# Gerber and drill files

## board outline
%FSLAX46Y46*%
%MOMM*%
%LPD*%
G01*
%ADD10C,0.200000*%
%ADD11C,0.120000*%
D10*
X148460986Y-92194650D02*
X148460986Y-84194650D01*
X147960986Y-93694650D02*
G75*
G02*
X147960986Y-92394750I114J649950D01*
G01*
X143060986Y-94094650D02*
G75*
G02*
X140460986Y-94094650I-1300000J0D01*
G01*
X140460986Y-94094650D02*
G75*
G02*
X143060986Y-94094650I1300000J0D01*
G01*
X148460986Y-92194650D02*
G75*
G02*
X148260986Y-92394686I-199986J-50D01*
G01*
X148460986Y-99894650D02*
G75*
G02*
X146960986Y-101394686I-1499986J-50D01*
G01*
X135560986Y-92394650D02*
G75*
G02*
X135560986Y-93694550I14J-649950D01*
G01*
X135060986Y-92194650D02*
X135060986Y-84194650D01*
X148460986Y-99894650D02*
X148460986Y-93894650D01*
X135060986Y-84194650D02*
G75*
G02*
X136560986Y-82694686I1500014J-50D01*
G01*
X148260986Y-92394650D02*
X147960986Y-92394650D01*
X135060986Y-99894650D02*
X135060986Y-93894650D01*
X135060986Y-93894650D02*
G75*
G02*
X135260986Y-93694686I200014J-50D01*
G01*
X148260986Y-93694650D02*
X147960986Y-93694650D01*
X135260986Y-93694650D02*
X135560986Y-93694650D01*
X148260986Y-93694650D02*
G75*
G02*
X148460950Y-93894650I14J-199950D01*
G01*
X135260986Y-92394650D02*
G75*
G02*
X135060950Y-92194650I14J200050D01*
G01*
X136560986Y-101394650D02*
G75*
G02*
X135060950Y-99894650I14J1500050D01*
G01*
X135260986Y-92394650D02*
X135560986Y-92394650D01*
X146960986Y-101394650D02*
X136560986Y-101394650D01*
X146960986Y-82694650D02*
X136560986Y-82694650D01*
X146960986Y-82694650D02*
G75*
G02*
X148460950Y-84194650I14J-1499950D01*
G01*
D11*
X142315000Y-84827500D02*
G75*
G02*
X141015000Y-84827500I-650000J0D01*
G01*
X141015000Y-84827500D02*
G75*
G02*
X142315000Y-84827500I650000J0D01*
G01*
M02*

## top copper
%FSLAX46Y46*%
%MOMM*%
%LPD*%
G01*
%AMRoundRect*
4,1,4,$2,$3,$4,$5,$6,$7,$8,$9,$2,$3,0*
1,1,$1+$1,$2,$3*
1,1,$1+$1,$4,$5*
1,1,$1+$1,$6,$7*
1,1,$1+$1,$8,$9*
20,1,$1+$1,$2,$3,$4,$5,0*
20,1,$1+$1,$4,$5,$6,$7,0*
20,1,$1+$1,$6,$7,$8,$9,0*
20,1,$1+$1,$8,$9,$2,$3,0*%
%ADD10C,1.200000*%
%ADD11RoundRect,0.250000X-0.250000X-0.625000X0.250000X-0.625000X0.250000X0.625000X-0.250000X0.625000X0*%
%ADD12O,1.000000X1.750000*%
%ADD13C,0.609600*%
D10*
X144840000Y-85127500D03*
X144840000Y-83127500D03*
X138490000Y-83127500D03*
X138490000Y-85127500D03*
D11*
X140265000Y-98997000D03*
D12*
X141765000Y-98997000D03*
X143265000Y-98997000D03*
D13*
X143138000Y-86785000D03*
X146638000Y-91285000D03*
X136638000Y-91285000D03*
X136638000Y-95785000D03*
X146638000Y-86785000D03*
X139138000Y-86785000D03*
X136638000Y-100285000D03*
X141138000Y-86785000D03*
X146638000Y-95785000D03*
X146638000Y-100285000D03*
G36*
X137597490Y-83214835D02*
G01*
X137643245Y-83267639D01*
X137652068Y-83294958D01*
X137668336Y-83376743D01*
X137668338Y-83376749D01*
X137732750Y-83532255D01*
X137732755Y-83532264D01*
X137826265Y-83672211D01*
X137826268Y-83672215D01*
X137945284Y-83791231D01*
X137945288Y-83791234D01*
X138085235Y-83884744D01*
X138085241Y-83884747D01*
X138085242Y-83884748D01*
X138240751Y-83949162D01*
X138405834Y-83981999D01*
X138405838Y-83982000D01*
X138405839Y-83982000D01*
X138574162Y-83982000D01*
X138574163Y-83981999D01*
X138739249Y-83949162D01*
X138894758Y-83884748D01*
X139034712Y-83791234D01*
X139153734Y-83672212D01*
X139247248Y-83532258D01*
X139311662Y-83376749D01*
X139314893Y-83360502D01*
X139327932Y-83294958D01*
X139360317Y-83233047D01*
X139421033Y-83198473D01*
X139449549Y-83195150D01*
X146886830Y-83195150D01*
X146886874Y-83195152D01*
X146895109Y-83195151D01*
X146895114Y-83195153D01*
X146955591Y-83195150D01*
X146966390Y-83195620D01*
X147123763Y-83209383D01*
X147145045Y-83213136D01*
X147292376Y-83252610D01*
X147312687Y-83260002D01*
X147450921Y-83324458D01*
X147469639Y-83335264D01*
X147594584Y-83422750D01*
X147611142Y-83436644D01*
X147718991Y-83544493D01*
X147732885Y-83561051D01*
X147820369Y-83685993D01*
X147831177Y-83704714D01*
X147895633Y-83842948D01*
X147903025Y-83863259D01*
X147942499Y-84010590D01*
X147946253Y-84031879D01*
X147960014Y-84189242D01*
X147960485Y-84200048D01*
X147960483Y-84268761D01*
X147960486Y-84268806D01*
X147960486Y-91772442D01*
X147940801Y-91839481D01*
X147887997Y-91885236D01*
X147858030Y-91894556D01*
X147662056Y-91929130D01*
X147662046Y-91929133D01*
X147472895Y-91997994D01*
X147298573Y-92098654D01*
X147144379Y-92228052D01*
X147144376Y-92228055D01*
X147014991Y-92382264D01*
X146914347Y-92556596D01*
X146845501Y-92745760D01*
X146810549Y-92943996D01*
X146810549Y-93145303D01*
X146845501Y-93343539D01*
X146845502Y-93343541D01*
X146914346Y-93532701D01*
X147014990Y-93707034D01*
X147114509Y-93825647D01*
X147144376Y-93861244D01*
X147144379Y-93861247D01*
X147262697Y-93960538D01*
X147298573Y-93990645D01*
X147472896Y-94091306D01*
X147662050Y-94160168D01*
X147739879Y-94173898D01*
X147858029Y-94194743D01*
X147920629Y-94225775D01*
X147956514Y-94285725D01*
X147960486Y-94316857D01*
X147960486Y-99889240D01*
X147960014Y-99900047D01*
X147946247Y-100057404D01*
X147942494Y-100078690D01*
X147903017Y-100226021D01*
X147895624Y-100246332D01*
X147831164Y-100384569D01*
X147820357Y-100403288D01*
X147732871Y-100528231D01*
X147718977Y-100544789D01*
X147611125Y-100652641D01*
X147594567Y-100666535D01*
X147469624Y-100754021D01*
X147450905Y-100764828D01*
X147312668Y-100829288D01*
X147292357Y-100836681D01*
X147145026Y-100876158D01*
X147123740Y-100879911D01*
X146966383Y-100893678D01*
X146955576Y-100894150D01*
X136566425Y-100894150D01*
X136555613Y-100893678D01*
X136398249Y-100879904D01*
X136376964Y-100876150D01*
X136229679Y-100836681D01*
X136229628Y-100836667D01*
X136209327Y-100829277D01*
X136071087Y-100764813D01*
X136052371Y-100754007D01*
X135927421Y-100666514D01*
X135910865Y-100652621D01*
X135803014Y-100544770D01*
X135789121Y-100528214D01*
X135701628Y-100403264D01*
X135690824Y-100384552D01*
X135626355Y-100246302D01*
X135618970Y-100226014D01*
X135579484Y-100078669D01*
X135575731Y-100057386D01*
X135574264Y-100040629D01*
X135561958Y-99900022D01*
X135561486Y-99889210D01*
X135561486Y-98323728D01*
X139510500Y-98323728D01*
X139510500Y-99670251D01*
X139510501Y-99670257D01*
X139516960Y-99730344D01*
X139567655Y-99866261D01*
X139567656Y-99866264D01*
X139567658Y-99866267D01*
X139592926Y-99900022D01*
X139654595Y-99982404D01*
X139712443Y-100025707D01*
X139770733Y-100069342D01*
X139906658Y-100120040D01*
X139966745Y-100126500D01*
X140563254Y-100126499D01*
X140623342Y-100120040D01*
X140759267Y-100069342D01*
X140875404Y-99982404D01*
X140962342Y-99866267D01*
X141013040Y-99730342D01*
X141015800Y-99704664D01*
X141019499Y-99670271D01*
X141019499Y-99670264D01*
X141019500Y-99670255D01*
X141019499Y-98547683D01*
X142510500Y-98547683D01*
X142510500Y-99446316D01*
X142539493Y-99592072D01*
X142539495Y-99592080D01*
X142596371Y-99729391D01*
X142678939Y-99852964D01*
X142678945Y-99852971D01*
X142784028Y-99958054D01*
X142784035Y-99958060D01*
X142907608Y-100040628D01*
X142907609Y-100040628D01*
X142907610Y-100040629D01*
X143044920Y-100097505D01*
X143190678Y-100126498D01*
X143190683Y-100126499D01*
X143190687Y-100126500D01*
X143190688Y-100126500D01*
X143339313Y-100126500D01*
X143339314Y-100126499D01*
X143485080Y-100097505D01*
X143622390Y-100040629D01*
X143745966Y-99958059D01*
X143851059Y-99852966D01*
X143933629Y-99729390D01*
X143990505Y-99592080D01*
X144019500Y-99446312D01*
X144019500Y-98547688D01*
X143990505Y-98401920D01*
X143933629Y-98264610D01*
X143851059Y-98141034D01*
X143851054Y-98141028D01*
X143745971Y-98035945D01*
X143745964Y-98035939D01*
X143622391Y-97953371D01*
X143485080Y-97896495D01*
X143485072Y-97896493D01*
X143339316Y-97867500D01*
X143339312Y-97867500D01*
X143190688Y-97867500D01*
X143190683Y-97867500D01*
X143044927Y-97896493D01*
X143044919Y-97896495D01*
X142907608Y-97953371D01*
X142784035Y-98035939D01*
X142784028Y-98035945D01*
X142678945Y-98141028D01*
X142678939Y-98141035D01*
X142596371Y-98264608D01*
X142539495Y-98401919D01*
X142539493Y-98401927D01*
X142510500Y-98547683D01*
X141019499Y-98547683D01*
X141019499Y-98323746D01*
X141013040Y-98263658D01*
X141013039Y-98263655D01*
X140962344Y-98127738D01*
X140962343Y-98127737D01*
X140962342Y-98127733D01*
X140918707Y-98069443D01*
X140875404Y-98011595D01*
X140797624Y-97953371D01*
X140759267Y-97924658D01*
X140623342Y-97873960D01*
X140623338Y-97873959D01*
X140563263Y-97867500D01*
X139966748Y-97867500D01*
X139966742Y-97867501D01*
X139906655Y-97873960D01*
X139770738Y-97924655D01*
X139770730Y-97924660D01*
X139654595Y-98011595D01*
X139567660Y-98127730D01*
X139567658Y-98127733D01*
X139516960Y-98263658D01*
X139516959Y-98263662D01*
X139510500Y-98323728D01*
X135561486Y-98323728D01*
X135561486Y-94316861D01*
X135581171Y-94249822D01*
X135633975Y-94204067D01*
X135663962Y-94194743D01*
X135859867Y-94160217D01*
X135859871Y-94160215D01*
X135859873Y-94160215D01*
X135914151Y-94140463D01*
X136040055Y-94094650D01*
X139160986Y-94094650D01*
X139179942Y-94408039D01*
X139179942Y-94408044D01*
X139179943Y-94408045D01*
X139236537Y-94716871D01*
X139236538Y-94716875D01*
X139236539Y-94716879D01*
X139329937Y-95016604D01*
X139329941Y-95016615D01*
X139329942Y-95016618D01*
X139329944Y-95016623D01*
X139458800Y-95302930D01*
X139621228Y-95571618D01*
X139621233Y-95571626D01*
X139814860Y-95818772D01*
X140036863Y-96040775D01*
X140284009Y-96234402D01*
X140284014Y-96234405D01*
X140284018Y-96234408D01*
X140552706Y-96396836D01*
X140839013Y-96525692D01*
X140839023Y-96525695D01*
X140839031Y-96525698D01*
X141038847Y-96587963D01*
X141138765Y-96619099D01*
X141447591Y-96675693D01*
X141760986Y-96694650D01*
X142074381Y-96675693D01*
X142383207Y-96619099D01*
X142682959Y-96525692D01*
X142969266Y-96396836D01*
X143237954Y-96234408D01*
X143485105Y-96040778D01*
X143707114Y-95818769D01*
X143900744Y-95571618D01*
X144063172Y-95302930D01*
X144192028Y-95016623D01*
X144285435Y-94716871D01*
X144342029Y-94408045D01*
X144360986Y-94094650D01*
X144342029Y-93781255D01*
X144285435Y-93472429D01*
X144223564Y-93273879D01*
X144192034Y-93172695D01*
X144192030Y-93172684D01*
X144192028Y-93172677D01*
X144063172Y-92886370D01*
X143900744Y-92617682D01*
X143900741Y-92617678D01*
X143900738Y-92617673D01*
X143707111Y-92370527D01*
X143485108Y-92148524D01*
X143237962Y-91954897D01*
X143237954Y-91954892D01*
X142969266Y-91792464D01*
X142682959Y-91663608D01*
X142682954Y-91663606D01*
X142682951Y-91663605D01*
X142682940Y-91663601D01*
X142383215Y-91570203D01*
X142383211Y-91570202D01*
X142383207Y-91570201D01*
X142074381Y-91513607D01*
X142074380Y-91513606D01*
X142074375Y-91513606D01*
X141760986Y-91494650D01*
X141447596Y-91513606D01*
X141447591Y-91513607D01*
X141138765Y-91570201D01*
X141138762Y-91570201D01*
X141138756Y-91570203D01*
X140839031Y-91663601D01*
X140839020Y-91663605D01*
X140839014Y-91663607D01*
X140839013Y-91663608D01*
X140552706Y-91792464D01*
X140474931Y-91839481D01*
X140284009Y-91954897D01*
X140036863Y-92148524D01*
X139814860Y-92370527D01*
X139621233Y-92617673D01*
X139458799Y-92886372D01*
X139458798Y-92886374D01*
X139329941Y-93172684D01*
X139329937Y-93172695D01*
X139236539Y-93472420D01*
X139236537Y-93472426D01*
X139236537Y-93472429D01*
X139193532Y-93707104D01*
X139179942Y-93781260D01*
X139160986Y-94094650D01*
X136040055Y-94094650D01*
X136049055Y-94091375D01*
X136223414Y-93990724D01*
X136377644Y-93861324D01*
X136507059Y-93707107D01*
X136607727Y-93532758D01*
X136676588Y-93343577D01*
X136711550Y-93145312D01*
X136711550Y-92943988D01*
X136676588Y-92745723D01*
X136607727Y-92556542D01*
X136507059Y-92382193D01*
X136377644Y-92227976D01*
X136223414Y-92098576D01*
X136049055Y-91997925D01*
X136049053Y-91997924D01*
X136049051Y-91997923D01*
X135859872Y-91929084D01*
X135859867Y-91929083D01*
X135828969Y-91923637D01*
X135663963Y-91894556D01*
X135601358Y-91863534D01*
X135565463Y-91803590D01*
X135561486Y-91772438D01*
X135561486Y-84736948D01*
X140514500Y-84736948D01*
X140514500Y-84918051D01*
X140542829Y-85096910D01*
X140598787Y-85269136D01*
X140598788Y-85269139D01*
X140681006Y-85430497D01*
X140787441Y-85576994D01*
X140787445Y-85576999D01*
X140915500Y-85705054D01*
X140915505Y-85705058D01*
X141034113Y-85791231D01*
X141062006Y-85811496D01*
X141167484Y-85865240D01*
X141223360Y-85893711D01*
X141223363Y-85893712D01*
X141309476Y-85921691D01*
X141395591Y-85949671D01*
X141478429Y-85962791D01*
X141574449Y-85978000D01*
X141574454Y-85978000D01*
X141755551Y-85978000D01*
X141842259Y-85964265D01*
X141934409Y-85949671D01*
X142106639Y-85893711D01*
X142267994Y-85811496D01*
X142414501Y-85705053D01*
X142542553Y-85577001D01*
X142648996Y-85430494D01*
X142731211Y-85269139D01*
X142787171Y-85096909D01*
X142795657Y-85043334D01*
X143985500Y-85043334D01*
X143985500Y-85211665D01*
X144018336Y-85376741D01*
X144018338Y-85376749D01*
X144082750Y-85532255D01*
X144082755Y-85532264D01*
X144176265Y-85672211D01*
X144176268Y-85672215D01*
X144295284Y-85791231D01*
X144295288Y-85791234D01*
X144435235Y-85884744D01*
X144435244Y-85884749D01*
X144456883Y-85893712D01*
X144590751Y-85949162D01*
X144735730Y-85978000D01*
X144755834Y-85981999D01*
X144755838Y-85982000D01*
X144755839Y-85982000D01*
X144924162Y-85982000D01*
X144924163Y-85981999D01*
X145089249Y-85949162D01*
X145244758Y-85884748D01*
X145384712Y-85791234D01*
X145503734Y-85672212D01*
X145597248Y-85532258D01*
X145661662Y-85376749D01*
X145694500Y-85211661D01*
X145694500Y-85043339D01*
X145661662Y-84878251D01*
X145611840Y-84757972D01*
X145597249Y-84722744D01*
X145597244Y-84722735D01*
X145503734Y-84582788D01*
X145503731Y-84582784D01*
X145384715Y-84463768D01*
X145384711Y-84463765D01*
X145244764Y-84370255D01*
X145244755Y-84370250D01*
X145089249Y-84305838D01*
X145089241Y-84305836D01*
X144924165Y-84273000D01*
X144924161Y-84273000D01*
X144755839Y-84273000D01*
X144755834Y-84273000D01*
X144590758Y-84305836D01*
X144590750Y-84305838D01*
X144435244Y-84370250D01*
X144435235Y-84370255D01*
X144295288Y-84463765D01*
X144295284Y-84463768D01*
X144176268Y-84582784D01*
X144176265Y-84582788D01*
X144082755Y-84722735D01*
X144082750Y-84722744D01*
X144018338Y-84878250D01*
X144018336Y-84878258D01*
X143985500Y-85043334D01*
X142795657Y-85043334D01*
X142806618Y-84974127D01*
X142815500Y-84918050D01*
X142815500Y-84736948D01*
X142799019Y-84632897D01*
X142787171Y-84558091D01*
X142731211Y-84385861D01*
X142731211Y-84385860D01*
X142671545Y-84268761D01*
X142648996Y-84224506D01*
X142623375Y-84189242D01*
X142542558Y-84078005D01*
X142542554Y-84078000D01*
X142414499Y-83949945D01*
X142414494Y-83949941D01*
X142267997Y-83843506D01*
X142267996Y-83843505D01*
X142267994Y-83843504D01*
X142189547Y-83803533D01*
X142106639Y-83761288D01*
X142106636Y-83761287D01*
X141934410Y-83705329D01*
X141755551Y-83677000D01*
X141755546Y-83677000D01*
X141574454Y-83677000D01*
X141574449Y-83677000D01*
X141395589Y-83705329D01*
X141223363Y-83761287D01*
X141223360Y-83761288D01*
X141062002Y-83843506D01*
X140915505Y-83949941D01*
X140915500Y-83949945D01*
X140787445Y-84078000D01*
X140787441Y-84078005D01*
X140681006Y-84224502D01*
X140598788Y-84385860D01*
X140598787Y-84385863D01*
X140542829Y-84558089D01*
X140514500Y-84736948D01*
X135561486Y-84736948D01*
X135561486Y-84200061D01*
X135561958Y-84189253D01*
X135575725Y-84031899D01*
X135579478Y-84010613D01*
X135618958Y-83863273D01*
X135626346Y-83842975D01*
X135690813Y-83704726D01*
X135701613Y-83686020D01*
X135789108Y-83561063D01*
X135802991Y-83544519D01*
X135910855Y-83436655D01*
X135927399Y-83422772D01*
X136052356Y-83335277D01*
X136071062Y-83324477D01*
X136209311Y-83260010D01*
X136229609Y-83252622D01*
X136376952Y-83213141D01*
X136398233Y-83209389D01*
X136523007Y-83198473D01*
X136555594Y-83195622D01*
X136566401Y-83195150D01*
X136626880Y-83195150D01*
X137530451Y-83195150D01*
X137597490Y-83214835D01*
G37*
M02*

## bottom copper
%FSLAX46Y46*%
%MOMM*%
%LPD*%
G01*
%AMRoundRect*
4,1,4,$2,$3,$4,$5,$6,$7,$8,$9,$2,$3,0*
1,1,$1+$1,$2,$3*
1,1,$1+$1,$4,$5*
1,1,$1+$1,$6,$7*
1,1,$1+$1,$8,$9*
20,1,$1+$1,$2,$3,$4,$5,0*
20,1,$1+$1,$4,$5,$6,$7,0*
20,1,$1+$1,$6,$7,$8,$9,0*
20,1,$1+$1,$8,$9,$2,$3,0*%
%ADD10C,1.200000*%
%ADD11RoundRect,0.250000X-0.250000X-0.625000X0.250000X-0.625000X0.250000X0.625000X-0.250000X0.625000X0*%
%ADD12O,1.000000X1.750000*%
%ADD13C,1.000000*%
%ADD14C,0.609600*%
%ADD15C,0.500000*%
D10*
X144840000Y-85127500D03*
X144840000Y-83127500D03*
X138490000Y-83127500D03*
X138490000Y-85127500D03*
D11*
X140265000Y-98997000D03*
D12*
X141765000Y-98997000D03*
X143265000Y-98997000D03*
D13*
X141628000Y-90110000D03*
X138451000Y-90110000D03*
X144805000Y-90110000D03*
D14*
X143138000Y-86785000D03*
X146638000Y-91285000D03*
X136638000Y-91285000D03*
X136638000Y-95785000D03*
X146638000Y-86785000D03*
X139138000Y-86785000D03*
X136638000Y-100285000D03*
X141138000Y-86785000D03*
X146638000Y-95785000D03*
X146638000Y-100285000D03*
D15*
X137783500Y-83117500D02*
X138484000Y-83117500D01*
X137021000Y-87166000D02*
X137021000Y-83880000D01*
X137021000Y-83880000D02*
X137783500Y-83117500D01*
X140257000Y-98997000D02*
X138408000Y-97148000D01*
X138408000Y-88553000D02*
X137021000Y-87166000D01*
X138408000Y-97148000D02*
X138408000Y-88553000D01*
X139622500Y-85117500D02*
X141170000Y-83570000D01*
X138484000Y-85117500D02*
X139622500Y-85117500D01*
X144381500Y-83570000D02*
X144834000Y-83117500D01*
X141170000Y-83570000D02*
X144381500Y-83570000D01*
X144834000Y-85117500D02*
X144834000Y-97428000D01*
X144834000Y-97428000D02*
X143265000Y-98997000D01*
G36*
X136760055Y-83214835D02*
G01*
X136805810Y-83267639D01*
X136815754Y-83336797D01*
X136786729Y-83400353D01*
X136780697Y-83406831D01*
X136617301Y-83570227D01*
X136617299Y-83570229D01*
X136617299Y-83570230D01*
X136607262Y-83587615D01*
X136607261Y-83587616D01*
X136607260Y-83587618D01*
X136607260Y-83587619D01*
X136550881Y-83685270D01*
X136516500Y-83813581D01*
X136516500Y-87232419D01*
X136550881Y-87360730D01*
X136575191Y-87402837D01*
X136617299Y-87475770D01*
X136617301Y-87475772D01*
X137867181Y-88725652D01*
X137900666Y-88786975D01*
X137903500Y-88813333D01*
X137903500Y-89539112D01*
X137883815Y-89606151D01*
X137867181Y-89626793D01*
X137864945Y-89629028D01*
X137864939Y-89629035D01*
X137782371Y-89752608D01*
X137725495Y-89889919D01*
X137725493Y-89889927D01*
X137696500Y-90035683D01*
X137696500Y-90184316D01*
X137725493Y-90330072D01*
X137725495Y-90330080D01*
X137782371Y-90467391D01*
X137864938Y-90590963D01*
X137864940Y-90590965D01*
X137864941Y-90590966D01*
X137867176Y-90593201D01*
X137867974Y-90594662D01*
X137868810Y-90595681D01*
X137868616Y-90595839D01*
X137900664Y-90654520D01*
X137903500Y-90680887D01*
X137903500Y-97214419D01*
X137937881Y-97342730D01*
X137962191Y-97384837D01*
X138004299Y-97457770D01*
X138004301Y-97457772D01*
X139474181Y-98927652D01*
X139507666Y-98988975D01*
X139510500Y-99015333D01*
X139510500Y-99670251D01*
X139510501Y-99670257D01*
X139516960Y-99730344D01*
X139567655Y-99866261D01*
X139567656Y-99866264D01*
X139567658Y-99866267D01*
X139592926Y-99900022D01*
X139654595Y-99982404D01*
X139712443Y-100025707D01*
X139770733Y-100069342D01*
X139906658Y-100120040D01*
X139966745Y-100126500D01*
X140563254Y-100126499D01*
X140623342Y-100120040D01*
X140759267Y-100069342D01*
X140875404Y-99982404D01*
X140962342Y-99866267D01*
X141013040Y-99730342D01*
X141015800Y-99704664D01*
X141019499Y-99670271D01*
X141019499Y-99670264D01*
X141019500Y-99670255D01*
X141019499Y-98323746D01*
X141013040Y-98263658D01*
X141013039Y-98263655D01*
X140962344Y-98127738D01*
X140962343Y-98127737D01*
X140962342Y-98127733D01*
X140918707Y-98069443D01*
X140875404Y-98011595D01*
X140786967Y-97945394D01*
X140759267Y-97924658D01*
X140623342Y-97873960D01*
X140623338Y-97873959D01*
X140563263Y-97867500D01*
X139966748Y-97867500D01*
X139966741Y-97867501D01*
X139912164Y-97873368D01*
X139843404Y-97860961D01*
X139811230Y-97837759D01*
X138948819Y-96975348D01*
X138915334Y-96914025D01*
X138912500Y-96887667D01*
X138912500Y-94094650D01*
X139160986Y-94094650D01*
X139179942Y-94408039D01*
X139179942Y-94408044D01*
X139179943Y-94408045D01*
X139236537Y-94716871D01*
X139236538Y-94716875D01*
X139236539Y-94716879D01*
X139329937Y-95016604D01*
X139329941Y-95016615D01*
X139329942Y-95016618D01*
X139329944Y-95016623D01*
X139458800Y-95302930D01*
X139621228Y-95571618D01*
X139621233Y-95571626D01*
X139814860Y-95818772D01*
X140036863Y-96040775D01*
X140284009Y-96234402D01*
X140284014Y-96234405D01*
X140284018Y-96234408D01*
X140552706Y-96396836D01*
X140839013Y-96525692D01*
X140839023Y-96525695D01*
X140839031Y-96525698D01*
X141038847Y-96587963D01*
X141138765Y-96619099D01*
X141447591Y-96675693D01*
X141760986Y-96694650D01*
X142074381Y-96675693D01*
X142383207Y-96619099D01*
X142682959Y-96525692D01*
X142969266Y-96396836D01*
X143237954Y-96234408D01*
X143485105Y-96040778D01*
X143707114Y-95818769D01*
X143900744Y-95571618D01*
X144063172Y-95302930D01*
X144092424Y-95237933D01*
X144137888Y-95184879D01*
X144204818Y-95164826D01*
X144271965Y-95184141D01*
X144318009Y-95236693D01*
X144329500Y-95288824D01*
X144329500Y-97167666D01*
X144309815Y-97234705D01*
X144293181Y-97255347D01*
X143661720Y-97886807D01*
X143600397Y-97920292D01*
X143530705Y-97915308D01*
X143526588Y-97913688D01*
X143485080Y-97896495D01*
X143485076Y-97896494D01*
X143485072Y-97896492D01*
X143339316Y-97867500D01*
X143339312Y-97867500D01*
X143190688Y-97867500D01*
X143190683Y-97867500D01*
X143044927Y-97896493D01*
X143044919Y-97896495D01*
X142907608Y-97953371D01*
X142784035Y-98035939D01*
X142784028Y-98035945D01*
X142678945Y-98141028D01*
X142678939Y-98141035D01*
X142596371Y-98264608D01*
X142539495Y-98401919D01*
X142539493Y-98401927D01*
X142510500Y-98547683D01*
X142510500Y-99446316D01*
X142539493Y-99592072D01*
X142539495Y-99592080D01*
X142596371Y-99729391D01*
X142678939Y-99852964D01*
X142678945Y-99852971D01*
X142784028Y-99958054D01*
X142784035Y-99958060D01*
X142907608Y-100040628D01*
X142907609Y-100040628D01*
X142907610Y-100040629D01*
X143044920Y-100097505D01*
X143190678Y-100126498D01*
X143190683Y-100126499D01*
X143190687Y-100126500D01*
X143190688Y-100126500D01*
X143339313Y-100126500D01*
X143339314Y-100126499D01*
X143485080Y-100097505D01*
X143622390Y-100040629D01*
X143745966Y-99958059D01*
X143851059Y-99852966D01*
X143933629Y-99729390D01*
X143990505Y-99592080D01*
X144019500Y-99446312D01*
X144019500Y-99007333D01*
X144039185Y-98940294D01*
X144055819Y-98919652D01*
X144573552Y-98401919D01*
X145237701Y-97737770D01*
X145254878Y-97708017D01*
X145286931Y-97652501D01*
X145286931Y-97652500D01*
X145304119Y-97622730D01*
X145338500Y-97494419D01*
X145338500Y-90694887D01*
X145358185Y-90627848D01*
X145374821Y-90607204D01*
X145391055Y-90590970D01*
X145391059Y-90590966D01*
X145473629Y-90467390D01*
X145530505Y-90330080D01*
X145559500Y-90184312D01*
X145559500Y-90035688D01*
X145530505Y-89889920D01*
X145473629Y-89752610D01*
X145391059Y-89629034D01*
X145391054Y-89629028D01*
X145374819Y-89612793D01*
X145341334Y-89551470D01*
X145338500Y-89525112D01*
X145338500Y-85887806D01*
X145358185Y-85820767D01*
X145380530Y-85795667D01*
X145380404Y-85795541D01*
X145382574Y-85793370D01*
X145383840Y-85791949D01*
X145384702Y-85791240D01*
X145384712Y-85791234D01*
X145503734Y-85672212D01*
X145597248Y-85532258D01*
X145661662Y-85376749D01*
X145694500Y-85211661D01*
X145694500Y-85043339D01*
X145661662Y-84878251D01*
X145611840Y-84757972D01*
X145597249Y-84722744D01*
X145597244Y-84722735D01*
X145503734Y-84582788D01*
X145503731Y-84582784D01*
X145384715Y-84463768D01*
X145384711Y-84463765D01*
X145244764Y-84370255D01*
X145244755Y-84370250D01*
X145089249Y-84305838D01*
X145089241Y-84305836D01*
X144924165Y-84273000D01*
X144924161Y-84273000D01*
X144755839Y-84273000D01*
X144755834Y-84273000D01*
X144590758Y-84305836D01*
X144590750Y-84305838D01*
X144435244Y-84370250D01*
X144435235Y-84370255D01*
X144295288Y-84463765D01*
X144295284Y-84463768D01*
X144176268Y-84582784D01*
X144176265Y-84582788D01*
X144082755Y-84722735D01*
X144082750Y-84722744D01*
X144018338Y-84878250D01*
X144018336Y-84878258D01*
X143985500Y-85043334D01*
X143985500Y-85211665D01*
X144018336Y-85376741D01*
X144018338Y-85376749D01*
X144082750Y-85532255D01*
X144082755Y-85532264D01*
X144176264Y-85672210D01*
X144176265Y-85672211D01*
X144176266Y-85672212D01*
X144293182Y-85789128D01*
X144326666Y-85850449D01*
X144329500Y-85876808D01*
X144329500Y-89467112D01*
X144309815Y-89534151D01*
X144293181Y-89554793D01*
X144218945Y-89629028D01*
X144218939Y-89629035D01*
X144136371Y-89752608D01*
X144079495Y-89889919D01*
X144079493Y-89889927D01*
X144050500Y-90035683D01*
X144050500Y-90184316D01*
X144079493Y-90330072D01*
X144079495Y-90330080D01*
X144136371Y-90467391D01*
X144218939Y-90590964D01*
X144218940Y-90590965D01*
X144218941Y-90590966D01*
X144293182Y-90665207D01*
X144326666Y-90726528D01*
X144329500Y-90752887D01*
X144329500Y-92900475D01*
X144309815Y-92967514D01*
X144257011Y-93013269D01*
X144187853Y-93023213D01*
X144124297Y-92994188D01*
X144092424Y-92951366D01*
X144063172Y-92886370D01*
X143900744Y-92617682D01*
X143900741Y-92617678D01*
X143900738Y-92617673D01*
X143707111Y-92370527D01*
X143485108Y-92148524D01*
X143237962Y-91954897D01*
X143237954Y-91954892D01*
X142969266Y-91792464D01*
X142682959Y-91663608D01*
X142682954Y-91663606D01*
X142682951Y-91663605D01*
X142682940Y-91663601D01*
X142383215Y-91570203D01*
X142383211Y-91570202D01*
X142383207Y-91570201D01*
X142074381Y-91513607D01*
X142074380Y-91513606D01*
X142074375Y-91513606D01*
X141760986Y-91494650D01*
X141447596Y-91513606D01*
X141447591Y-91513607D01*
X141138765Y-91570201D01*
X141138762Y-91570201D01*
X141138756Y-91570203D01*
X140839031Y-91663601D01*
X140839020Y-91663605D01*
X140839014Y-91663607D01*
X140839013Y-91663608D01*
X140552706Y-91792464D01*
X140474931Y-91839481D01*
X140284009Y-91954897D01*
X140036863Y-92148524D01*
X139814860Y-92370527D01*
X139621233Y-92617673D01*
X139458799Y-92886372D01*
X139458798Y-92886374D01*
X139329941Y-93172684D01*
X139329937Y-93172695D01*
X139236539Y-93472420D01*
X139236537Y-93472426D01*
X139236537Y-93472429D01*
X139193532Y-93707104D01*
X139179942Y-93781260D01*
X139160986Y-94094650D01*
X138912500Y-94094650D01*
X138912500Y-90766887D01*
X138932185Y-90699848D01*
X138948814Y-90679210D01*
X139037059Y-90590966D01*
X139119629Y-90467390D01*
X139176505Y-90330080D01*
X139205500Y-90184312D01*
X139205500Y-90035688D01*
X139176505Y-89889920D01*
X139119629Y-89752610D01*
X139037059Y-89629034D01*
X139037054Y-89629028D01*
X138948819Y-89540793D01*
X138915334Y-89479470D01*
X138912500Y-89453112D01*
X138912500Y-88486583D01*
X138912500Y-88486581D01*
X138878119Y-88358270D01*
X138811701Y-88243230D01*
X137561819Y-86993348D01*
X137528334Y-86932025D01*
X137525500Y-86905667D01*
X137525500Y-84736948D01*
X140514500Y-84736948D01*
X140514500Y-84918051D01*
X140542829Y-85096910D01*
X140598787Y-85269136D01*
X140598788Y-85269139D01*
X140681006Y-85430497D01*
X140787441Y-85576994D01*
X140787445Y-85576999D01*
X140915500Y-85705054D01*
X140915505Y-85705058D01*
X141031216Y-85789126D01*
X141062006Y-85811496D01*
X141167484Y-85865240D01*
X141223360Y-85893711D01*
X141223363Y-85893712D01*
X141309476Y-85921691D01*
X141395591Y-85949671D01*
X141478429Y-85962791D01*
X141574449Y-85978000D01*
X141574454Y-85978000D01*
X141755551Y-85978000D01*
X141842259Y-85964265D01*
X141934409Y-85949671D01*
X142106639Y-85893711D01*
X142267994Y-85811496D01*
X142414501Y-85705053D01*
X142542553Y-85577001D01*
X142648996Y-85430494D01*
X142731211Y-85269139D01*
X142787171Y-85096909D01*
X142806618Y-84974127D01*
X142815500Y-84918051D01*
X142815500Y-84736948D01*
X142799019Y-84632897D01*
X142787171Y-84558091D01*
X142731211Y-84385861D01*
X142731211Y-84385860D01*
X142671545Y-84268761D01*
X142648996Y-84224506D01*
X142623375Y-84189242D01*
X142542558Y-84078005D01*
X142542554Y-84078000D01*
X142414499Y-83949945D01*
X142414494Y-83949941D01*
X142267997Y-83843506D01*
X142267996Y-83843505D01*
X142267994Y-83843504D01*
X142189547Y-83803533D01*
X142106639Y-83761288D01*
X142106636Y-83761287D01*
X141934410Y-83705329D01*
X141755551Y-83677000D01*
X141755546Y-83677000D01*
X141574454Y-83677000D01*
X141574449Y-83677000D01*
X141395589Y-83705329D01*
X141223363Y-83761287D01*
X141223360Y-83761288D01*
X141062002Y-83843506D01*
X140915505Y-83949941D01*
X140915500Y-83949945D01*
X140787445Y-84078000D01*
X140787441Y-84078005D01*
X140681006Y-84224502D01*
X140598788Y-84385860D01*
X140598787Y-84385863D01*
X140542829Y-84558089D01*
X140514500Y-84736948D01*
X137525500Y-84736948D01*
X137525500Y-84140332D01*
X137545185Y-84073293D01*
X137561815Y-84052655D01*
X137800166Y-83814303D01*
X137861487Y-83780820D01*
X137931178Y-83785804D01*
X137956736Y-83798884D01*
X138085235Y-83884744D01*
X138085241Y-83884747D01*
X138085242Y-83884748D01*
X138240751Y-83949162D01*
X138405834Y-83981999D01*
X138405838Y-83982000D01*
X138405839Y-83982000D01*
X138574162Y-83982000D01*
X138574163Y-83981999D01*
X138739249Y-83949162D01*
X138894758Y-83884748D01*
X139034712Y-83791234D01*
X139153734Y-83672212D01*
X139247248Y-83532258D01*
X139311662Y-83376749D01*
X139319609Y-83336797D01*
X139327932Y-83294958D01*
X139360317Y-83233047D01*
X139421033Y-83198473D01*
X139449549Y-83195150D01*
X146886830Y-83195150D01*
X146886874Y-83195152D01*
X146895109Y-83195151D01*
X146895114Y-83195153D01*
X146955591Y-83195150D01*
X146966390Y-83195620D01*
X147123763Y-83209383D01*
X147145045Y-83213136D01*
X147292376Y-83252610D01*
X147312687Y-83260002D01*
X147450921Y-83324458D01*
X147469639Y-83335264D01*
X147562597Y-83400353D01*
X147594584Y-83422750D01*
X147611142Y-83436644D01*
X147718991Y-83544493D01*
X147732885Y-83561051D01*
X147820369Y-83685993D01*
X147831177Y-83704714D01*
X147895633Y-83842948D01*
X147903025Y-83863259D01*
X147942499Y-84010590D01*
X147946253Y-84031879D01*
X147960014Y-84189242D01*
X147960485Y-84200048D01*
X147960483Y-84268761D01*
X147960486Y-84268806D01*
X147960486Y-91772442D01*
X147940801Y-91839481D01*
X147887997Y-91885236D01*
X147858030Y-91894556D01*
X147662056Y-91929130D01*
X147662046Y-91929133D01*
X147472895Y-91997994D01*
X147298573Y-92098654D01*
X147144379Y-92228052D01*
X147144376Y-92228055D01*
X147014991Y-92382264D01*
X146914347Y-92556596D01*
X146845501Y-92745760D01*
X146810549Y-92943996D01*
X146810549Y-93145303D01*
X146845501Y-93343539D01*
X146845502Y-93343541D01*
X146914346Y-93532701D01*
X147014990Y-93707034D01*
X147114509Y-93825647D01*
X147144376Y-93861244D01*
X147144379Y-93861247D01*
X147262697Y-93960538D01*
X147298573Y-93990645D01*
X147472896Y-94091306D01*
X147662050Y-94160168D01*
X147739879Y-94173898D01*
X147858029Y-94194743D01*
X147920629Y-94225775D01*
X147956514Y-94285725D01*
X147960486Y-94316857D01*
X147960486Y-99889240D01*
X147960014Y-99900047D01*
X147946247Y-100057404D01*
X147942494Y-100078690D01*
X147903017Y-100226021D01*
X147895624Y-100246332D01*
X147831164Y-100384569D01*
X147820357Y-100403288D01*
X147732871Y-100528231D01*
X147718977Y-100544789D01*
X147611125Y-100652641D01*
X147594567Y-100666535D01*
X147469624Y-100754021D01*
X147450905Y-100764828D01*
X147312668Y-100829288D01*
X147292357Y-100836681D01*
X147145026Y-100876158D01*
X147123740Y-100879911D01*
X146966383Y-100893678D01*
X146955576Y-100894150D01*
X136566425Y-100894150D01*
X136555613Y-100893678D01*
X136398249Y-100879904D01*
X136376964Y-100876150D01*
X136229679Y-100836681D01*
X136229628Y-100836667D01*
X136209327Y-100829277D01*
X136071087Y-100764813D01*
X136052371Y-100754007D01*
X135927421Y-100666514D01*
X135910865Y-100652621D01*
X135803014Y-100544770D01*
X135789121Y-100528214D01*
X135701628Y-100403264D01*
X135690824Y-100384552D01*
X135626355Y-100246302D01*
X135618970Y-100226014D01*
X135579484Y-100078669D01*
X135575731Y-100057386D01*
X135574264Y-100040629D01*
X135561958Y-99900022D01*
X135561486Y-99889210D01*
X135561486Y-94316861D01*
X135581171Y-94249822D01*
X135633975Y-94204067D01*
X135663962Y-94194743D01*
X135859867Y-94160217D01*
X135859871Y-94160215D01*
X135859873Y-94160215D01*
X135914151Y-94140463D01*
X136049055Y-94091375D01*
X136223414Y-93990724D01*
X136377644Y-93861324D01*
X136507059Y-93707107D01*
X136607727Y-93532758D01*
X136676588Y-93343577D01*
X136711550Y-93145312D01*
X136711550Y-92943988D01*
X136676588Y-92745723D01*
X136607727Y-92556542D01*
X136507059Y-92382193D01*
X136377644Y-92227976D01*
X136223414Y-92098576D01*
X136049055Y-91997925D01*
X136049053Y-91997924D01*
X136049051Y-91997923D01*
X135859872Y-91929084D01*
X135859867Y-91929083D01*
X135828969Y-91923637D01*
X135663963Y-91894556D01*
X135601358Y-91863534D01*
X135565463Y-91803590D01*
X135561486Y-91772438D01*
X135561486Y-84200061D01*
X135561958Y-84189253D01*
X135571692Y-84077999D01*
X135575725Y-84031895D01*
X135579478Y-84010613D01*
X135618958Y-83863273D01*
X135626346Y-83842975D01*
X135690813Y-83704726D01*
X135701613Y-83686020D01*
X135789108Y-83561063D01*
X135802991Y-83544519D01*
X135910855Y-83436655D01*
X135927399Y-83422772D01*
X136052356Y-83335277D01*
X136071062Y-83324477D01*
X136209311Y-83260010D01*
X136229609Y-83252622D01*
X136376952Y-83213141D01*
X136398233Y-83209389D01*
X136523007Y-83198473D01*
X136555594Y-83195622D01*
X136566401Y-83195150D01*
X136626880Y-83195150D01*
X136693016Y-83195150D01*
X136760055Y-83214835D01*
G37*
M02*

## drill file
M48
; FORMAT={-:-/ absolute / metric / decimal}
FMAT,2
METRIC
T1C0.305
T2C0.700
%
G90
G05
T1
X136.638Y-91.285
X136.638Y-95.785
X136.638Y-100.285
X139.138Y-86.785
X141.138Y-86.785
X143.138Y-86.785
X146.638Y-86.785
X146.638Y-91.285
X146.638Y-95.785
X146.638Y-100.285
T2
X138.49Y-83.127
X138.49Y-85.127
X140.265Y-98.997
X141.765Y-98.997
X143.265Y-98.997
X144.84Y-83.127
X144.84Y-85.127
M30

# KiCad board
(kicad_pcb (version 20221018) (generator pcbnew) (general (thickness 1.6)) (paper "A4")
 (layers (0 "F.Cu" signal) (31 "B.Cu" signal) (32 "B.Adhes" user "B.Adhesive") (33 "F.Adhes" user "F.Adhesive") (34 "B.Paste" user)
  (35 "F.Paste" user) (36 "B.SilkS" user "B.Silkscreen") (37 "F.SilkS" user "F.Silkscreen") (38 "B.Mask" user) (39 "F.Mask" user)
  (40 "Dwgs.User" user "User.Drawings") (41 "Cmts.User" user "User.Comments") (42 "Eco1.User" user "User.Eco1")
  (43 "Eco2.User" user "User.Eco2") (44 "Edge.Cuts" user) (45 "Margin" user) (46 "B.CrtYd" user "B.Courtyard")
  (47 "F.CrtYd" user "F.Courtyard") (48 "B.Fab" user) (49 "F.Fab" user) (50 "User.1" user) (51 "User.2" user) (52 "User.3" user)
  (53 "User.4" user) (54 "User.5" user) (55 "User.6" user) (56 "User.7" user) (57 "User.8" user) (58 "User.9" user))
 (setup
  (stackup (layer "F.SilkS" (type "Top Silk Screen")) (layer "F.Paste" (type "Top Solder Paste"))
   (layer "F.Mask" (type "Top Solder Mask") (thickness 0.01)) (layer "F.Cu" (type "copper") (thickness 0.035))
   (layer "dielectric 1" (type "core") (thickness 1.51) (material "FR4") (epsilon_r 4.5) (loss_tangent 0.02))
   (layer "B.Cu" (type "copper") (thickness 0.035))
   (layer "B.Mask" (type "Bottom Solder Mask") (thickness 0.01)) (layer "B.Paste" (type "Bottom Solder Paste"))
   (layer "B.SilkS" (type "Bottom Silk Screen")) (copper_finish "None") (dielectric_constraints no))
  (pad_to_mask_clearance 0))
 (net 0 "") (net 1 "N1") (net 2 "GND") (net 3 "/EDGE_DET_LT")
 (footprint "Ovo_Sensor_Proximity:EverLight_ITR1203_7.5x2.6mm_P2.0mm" (layer "F.Cu") (at 141.665 84.1275 180)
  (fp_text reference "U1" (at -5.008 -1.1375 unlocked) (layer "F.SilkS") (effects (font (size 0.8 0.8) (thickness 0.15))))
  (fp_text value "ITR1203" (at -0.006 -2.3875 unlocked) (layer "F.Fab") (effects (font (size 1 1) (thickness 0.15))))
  (fp_circle (center 0 -0.7) (end 0.65 -0.7) (stroke (width 0.12) (type solid)) (fill none) (layer "Edge.Cuts"))
  (pad "1" thru_hole circle (at -3.175 -1 180) (size 1.2 1.2) (drill 0.7) (layers "*.Cu" "*.Mask") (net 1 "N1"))
  (pad "2" thru_hole circle (at -3.175 1 180) (size 1.2 1.2) (drill 0.7) (layers "*.Cu" "*.Mask") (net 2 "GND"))
  (pad "3" thru_hole circle (at 3.175 1 180) (size 1.2 1.2) (drill 0.7) (layers "*.Cu" "*.Mask") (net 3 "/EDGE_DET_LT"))
  (pad "4" thru_hole circle (at 3.175 -1 180) (size 1.2 1.2) (drill 0.7) (layers "*.Cu" "*.Mask") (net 2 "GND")))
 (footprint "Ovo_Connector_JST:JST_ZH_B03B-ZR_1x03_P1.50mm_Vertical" (layer "F.Cu") (at 140.265 98.997)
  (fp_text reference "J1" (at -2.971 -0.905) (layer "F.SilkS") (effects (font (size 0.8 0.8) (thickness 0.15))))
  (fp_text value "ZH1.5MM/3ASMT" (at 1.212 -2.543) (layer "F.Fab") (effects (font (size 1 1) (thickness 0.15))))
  (pad "1" thru_hole roundrect (at 0 0) (size 1 1.75) (drill 0.7) (layers "*.Cu" "*.Mask") (roundrect_rratio 0.25) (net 3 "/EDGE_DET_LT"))
  (pad "2" thru_hole oval (at 1.5 0) (size 1 1.75) (drill 0.7) (layers "*.Cu" "*.Mask") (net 2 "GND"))
  (pad "3" thru_hole oval (at 3 0) (size 1 1.75) (drill 0.7) (layers "*.Cu" "*.Mask") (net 1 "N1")))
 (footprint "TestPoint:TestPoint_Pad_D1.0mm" (layer "B.Cu") (at 141.628 90.11 180)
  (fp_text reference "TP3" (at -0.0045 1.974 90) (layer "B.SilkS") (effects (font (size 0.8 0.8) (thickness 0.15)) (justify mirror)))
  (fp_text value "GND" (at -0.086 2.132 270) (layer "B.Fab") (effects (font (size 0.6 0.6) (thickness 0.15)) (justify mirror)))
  (pad "1" smd circle (at 0 0 180) (size 1 1) (layers "B.Cu" "B.Mask") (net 2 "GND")))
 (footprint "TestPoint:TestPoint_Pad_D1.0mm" (layer "B.Cu") (at 138.451 90.11 180)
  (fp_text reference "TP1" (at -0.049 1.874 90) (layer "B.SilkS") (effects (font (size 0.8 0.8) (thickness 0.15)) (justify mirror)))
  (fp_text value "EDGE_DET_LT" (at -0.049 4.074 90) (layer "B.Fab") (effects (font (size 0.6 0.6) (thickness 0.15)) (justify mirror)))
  (pad "1" smd circle (at 0 0 180) (size 1 1) (layers "B.Cu" "B.Mask") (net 3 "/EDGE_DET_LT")))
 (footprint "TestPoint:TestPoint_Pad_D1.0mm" (layer "B.Cu") (at 144.805 90.11 180)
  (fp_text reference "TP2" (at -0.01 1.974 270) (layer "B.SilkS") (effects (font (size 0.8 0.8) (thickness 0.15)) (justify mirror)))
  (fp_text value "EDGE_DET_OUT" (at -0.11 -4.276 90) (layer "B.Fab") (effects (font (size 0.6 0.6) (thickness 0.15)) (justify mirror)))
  (pad "1" smd circle (at 0 0 180) (size 1 1) (layers "B.Cu" "B.Mask") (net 1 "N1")))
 (gr_line (start 148.460986 92.19465) (end 148.460986 84.19465) (stroke (width 0.2) (type solid)) (layer "Edge.Cuts"))
 (gr_arc (start 147.960986 93.69465) (mid 147.31105 93.0447) (end 147.960986 92.39465) (stroke (width 0.2) (type solid)) (layer "Edge.Cuts"))
 (gr_circle (center 141.760986 94.09465) (end 143.060986 94.09465) (stroke (width 0.2) (type solid)) (fill none) (layer "Edge.Cuts"))
 (gr_arc (start 148.460986 92.19465) (mid 148.402418 92.336063) (end 148.260986 92.39465) (stroke (width 0.2) (type solid))
  (layer "Edge.Cuts"))
 (gr_arc (start 148.460986 99.89465) (mid 148.021657 100.955302) (end 146.960986 101.39465) (stroke (width 0.2) (type solid))
  (layer "Edge.Cuts"))
 (gr_arc (start 135.560986 92.39465) (mid 136.21105 93.0447) (end 135.560986 93.69465) (stroke (width 0.2) (type solid)) (layer "Edge.Cuts"))
 (gr_line (start 135.060986 92.19465) (end 135.060986 84.19465) (stroke (width 0.2) (type solid)) (layer "Edge.Cuts"))
 (gr_line (start 148.460986 99.89465) (end 148.460986 93.89465) (stroke (width 0.2) (type solid)) (layer "Edge.Cuts"))
 (gr_arc (start 135.060986 84.19465) (mid 135.500337 83.133982) (end 136.560986 82.69465) (stroke (width 0.2) (type solid))
  (layer "Edge.Cuts"))
 (gr_line (start 148.260986 92.39465) (end 147.960986 92.39465) (stroke (width 0.2) (type solid)) (layer "Edge.Cuts"))
 (gr_line (start 135.060986 99.89465) (end 135.060986 93.89465) (stroke (width 0.2) (type solid)) (layer "Edge.Cuts"))
 (gr_arc (start 135.060986 93.89465) (mid 135.119575 93.753221) (end 135.260986 93.69465) (stroke (width 0.2) (type solid))
  (layer "Edge.Cuts"))
 (gr_line (start 148.260986 93.69465) (end 147.960986 93.69465) (stroke (width 0.2) (type solid)) (layer "Edge.Cuts"))
 (gr_line (start 135.260986 93.69465) (end 135.560986 93.69465) (stroke (width 0.2) (type solid)) (layer "Edge.Cuts"))
 (gr_arc (start 148.260986 93.69465) (mid 148.402434 93.753221) (end 148.460986 93.89465) (stroke (width 0.2) (type solid))
  (layer "Edge.Cuts"))
 (gr_arc (start 135.260986 92.39465) (mid 135.119591 92.336063) (end 135.060986 92.19465) (stroke (width 0.2) (type solid))
  (layer "Edge.Cuts"))
 (gr_arc (start 136.560986 101.39465) (mid 135.500353 100.955302) (end 135.060986 99.89465) (stroke (width 0.2) (type solid))
  (layer "Edge.Cuts"))
 (gr_line (start 135.260986 92.39465) (end 135.560986 92.39465) (stroke (width 0.2) (type solid)) (layer "Edge.Cuts"))
 (gr_line (start 146.960986 101.39465) (end 136.560986 101.39465) (stroke (width 0.2) (type solid)) (layer "Edge.Cuts"))
 (gr_line (start 146.960986 82.69465) (end 136.560986 82.69465) (stroke (width 0.2) (type solid)) (layer "Edge.Cuts"))
 (gr_arc (start 146.960986 82.69465) (mid 148.021673 83.133982) (end 148.460986 84.19465) (stroke (width 0.2) (type solid))
  (layer "Edge.Cuts"))
 (segment (start 137.7835 83.1175) (end 138.484 83.1175) (width 0.5) (layer "B.Cu") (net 3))
 (segment (start 137.021 87.166) (end 137.021 83.88) (width 0.5) (layer "B.Cu") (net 3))
 (segment (start 137.021 83.88) (end 137.7835 83.1175) (width 0.5) (layer "B.Cu") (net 3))
 (segment (start 140.257 98.997) (end 138.408 97.148) (width 0.5) (layer "B.Cu") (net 3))
 (segment (start 138.408 88.553) (end 137.021 87.166) (width 0.5) (layer "B.Cu") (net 3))
 (segment (start 138.408 97.148) (end 138.408 88.553) (width 0.5) (layer "B.Cu") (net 3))
 (via (at 143.138 86.785) (size 0.6096) (drill 0.3048) (layers "F.Cu" "B.Cu") (free) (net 2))
 (via (at 146.638 91.285) (size 0.6096) (drill 0.3048) (layers "F.Cu" "B.Cu") (free) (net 2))
 (via (at 136.638 91.285) (size 0.6096) (drill 0.3048) (layers "F.Cu" "B.Cu") (free) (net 2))
 (via (at 136.638 95.785) (size 0.6096) (drill 0.3048) (layers "F.Cu" "B.Cu") (free) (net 2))
 (via (at 146.638 86.785) (size 0.6096) (drill 0.3048) (layers "F.Cu" "B.Cu") (free) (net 2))
 (via (at 139.138 86.785) (size 0.6096) (drill 0.3048) (layers "F.Cu" "B.Cu") (free) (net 2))
 (via (at 136.638 100.285) (size 0.6096) (drill 0.3048) (layers "F.Cu" "B.Cu") (free) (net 2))
 (via (at 141.138 86.785) (size 0.6096) (drill 0.3048) (layers "F.Cu" "B.Cu") (free) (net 2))
 (via (at 146.638 95.785) (size 0.6096) (drill 0.3048) (layers "F.Cu" "B.Cu") (free) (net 2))
 (via (at 146.638 100.285) (size 0.6096) (drill 0.3048) (layers "F.Cu" "B.Cu") (free) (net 2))
 (segment (start 139.6225 85.1175) (end 141.17 83.57) (width 0.5) (layer "B.Cu") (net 2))
 (segment (start 138.484 85.1175) (end 139.6225 85.1175) (width 0.5) (layer "B.Cu") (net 2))
 (segment (start 144.3815 83.57) (end 144.834 83.1175) (width 0.5) (layer "B.Cu") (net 2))
 (segment (start 141.17 83.57) (end 144.3815 83.57) (width 0.5) (layer "B.Cu") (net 2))
 (segment (start 144.834 85.1175) (end 144.834 97.428) (width 0.5) (layer "B.Cu") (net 1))
 (segment (start 144.834 97.428) (end 143.265 98.997) (width 0.5) (layer "B.Cu") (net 1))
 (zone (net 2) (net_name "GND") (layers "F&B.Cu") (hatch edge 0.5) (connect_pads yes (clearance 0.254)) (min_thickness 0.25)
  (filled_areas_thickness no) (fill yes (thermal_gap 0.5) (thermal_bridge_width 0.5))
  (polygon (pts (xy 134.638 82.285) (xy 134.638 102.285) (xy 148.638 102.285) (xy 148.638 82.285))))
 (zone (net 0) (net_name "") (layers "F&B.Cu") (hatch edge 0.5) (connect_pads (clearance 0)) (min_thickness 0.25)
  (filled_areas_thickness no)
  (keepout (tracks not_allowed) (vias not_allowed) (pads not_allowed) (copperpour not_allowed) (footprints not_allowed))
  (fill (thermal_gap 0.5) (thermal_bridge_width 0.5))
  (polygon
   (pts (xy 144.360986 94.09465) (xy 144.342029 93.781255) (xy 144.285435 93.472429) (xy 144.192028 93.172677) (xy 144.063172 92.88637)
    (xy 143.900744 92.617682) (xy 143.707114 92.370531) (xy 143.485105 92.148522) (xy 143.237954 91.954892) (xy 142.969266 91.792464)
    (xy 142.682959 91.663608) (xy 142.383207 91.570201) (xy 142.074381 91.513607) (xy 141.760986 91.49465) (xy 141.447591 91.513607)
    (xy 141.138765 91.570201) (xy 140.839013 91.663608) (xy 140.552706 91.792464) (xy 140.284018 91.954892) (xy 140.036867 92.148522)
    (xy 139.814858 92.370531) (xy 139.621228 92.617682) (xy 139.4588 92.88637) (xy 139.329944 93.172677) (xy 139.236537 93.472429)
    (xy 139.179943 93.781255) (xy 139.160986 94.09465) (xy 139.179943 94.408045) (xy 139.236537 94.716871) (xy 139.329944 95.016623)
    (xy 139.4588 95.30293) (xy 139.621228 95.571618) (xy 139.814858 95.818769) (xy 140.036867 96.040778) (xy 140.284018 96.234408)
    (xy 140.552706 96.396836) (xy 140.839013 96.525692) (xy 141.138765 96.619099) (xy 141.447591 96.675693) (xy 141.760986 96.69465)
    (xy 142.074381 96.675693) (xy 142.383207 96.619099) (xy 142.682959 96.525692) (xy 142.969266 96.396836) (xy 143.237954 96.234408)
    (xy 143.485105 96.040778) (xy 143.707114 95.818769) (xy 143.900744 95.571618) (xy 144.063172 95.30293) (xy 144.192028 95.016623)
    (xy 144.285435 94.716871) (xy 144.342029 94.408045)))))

